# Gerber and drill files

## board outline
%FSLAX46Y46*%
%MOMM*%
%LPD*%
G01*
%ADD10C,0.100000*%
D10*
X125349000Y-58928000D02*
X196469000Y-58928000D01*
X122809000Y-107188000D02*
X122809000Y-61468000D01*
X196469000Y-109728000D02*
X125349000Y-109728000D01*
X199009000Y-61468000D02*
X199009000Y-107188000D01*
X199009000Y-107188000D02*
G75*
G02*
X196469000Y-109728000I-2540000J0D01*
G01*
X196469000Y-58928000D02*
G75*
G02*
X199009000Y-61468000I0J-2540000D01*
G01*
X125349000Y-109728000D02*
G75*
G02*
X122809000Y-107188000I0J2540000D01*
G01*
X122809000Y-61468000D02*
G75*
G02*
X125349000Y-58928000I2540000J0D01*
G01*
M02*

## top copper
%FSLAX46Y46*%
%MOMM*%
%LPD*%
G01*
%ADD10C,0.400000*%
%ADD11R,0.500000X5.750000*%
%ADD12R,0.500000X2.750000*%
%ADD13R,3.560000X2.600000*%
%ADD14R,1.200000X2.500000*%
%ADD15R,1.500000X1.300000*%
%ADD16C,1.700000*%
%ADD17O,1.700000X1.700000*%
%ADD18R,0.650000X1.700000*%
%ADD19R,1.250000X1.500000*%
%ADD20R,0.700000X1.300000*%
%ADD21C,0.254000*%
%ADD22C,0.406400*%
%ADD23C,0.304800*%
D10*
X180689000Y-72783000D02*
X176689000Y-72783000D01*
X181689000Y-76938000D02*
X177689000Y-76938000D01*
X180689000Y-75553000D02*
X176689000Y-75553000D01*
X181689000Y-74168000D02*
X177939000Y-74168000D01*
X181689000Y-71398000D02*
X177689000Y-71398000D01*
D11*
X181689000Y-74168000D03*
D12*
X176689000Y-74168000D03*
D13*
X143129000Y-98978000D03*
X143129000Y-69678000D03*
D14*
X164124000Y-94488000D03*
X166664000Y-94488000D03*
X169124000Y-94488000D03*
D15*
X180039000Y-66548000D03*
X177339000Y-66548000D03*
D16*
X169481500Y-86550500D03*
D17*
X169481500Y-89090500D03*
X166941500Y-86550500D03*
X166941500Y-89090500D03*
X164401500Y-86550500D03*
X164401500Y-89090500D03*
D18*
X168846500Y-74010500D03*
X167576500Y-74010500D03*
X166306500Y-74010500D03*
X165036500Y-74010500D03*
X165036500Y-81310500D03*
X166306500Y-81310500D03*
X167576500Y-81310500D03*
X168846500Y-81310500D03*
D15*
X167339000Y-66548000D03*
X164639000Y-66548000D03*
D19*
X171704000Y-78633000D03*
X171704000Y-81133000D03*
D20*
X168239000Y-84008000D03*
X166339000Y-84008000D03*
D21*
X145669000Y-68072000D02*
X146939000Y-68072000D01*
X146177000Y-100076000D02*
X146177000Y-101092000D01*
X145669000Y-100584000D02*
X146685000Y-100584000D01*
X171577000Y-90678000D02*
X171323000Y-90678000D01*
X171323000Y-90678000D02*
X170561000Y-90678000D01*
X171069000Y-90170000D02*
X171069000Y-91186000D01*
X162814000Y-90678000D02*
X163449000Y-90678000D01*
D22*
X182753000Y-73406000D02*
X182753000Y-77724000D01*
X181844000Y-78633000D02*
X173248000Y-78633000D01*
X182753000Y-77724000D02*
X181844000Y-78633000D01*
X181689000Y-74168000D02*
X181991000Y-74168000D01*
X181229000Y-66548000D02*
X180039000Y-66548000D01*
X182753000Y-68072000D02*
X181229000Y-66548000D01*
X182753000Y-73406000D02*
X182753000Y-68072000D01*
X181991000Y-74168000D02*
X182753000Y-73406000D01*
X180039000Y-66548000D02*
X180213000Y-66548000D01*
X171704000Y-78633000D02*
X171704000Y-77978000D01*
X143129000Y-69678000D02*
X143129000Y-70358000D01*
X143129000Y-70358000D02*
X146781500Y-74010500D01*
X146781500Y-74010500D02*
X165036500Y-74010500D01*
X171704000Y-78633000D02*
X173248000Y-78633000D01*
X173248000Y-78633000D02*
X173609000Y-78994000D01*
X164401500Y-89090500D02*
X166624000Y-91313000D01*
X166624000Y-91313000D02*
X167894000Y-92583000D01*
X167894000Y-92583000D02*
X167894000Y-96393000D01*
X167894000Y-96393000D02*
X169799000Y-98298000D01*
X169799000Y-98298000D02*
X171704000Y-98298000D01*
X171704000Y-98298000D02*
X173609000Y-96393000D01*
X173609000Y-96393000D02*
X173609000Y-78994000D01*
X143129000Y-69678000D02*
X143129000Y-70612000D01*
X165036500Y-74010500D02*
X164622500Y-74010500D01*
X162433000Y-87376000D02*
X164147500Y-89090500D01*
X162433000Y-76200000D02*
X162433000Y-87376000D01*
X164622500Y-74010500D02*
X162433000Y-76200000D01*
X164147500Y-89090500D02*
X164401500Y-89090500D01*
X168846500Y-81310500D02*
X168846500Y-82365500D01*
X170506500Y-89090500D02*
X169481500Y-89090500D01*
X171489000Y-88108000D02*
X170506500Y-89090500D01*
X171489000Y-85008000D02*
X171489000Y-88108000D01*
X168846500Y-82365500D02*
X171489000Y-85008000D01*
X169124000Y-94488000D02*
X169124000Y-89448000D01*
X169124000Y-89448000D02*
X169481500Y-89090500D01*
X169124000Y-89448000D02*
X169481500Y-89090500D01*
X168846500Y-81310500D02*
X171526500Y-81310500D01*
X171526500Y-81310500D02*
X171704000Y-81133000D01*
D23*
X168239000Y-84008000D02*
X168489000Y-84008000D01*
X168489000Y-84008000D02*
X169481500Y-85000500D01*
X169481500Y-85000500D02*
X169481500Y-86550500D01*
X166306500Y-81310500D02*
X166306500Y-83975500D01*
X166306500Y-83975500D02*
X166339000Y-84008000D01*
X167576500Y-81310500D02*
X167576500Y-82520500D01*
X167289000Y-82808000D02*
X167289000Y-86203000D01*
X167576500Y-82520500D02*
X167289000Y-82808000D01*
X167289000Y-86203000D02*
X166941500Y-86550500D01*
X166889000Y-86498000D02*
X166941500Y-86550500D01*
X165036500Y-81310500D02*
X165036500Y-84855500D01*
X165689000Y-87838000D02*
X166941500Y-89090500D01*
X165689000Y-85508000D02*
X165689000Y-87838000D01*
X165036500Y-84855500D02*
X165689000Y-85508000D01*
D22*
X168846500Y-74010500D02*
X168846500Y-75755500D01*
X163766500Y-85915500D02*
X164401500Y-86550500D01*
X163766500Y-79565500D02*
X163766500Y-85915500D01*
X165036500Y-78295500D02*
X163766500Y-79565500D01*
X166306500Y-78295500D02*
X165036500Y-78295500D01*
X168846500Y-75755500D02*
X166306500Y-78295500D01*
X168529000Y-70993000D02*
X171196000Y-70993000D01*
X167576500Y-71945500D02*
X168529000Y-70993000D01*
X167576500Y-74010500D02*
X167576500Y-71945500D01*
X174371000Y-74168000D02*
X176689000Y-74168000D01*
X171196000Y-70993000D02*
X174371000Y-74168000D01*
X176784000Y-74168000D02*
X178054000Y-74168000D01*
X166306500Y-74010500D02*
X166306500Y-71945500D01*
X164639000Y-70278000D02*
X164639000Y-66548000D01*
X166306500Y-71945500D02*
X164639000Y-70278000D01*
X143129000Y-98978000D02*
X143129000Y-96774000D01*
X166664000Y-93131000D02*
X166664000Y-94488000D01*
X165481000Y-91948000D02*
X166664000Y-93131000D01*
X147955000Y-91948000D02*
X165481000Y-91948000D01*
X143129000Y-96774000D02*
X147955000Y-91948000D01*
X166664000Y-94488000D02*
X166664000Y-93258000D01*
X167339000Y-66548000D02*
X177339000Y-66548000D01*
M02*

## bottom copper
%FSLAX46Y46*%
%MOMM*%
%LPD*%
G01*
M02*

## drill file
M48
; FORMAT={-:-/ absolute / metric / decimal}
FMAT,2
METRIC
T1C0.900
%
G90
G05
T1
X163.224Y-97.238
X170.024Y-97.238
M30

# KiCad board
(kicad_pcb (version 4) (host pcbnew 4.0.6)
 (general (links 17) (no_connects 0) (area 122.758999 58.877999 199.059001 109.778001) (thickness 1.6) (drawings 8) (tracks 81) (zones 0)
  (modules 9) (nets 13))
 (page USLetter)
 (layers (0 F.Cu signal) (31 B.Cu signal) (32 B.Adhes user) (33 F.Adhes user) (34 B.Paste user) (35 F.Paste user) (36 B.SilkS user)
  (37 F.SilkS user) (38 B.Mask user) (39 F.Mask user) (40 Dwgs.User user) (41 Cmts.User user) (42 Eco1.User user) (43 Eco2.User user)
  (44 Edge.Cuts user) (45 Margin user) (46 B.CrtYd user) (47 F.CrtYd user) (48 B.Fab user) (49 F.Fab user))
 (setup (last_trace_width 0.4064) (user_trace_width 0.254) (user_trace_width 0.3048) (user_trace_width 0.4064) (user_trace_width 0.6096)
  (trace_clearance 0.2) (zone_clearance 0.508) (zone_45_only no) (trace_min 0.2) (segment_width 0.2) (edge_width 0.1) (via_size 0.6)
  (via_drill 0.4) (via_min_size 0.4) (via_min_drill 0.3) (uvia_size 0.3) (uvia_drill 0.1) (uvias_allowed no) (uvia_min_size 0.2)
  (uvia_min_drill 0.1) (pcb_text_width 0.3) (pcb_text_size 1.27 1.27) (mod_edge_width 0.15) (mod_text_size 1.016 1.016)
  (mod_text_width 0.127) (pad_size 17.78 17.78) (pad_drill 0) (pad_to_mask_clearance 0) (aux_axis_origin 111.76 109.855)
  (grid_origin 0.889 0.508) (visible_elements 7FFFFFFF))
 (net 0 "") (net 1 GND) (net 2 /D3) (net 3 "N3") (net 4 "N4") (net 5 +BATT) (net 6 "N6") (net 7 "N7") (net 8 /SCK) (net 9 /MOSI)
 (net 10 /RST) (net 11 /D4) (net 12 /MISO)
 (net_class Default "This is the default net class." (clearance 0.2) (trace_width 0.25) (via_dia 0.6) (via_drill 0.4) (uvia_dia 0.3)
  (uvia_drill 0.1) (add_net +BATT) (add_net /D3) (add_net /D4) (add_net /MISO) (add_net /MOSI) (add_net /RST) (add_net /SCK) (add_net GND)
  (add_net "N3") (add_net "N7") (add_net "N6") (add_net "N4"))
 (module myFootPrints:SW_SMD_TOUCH (layer F.Cu) (at 178.689 74.168 270)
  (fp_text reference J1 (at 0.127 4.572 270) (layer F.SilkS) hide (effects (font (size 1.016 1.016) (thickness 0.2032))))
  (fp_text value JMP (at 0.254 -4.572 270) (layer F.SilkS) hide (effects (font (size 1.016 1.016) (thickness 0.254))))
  (fp_line (start -1.385 -2) (end -1.385 2) (layer F.Cu) (width 0.4))
  (fp_line (start 2.77 -3) (end 2.77 1) (layer F.Cu) (width 0.4))
  (fp_line (start 1.385 -2) (end 1.385 2) (layer F.Cu) (width 0.4)) (fp_line (start 0 -3) (end 0 0.75) (layer F.Cu) (width 0.4))
  (fp_line (start -2.77 -3) (end -2.77 1) (layer F.Cu) (width 0.4))
  (pad 1 smd rect (at 0 -3 270) (size 5.75 0.5) (layers F.Cu F.Paste F.Mask) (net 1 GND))
  (pad 2 smd rect (at 0 2 270) (size 2.75 0.5) (layers F.Cu F.Paste F.Mask) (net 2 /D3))
  (pad 3 smd circle (at 0 -1 270) (size 3.5 3.5) (layers F.Paste F.Mask)))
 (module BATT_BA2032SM (layer F.Cu) (at 143.129 84.328 90)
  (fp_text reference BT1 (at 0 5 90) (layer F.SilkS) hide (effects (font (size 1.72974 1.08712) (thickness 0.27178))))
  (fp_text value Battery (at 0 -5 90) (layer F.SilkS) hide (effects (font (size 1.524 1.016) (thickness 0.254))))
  (pad 1 smd rect (at -14.65 0 90) (size 2.6 3.56) (layers F.Cu F.Paste F.Mask) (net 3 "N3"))
  (pad 2 smd rect (at 14.65 0 90) (size 2.6 3.56) (layers F.Cu F.Paste F.Mask) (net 1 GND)))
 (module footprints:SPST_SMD (layer F.Cu) (at 166.624 94.488)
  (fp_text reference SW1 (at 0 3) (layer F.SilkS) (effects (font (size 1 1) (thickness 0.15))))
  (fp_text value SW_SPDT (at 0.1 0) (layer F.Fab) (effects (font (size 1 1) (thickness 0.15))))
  (pad "" np_thru_hole circle (at 3.4 2.75) (size 0.9 0.9) (drill 0.9) (layers *.Cu *.Mask))
  (pad 1 smd rect (at -2.5 0) (size 1.2 2.5) (layers F.Cu F.Paste F.Mask) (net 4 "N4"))
  (pad 2 smd rect (at 0.04 0) (size 1.2 2.5) (layers F.Cu F.Paste F.Mask) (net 3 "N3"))
  (pad 3 smd rect (at 2.5 0) (size 1.2 2.5) (layers F.Cu F.Paste F.Mask) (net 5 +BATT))
  (pad "" np_thru_hole circle (at -3.4 2.75) (size 0.9 0.9) (drill 0.9) (layers *.Cu *.Mask)))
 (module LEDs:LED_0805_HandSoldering (layer F.Cu) (at 178.689 66.548 180)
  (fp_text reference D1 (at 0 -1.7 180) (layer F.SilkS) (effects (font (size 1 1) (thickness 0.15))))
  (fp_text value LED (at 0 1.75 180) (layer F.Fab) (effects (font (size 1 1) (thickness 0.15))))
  (pad 1 smd rect (at -1.35 0 180) (size 1.5 1.3) (layers F.Cu F.Paste F.Mask) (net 1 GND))
  (pad 2 smd rect (at 1.35 0 180) (size 1.5 1.3) (layers F.Cu F.Paste F.Mask) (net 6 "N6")))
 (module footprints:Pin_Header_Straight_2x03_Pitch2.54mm (layer F.Cu) (at 169.4815 86.5505 270)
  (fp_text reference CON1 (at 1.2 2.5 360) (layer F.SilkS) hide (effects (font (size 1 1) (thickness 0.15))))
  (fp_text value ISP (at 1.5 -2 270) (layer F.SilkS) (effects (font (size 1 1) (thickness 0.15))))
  (pad 1 smd circle (at 0 0 270) (size 1.7 1.7) (layers F.Cu F.Paste F.Mask) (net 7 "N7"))
  (pad 2 smd oval (at 2.54 0 270) (size 1.7 1.7) (layers F.Cu F.Paste F.Mask) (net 5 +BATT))
  (pad 3 smd oval (at 0 2.54 270) (size 1.7 1.7) (layers F.Cu F.Paste F.Mask) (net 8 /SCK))
  (pad 4 smd oval (at 2.54 2.54 270) (size 1.7 1.7) (layers F.Cu F.Paste F.Mask) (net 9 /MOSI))
  (pad 5 smd oval (at 0 5.08 270) (size 1.7 1.7) (layers F.Cu F.Paste F.Mask) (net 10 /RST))
  (pad 6 smd oval (at 2.54 5.08 270) (size 1.7 1.7) (layers F.Cu F.Paste F.Mask) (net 1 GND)))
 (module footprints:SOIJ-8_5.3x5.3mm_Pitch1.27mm (layer F.Cu) (at 166.9415 77.6605 270)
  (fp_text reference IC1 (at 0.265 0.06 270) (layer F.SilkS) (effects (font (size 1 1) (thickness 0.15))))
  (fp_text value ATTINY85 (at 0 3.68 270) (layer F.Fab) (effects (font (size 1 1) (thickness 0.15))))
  (pad 1 smd rect (at -3.65 -1.905 270) (size 1.7 0.65) (layers F.Cu F.Paste F.Mask) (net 10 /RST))
  (pad 2 smd rect (at -3.65 -0.635 270) (size 1.7 0.65) (layers F.Cu F.Paste F.Mask) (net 2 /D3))
  (pad 3 smd rect (at -3.65 0.635 270) (size 1.7 0.65) (layers F.Cu F.Paste F.Mask) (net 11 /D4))
  (pad 4 smd rect (at -3.65 1.905 270) (size 1.7 0.65) (layers F.Cu F.Paste F.Mask) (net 1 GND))
  (pad 5 smd rect (at 3.65 1.905 270) (size 1.7 0.65) (layers F.Cu F.Paste F.Mask) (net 9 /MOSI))
  (pad 6 smd rect (at 3.65 0.635 270) (size 1.7 0.65) (layers F.Cu F.Paste F.Mask) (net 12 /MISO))
  (pad 7 smd rect (at 3.65 -0.635 270) (size 1.7 0.65) (layers F.Cu F.Paste F.Mask) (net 8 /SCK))
  (pad 8 smd rect (at 3.65 -1.905 270) (size 1.7 0.65) (layers F.Cu F.Paste F.Mask) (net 5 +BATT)))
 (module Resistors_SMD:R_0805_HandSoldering (layer F.Cu) (at 165.989 66.548 180)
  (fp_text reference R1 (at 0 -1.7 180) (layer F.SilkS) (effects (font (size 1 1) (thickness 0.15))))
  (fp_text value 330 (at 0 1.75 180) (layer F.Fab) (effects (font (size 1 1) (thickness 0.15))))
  (pad 1 smd rect (at -1.35 0 180) (size 1.5 1.3) (layers F.Cu F.Paste F.Mask) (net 6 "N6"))
  (pad 2 smd rect (at 1.35 0 180) (size 1.5 1.3) (layers F.Cu F.Paste F.Mask) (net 11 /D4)))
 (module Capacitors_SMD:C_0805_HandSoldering (layer F.Cu) (at 171.704 79.883 270)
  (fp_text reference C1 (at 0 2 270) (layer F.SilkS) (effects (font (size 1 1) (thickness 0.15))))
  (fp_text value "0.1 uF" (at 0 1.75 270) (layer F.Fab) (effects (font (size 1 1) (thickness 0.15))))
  (pad 1 smd rect (at -1.25 0 270) (size 1.5 1.25) (layers F.Cu F.Paste F.Mask) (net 1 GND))
  (pad 2 smd rect (at 1.25 0 270) (size 1.5 1.25) (layers F.Cu F.Paste F.Mask) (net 5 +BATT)))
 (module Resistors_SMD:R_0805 (layer F.Cu) (at 167.289 84.008 180)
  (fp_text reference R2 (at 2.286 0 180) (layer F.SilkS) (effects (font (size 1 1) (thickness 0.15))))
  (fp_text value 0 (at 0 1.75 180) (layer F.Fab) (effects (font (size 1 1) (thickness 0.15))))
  (pad 1 smd rect (at -0.95 0 180) (size 0.7 1.3) (layers F.Cu F.Paste F.Mask) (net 7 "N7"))
  (pad 2 smd rect (at 0.95 0 180) (size 0.7 1.3) (layers F.Cu F.Paste F.Mask) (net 12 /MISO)))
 (gr_line (start 125.349 58.928) (end 196.469 58.928) (angle 90) (layer Edge.Cuts) (width 0.1))
 (gr_line (start 122.809 107.188) (end 122.809 61.468) (angle 90) (layer Edge.Cuts) (width 0.1))
 (gr_line (start 196.469 109.728) (end 125.349 109.728) (angle 90) (layer Edge.Cuts) (width 0.1))
 (gr_line (start 199.009 61.468) (end 199.009 107.188) (angle 90) (layer Edge.Cuts) (width 0.1))
 (gr_arc (start 196.469 107.188) (end 199.009 107.188) (angle 90) (layer Edge.Cuts) (width 0.1))
 (gr_arc (start 196.469 61.468) (end 196.469 58.928) (angle 90) (layer Edge.Cuts) (width 0.1))
 (gr_arc (start 125.349 107.188) (end 125.349 109.728) (angle 90) (layer Edge.Cuts) (width 0.1))
 (gr_arc (start 125.349 61.468) (end 122.809 61.468) (angle 90) (layer Edge.Cuts) (width 0.1))
 (segment (start 145.669 68.072) (end 146.939 68.072) (width 0.254) (layer F.Cu) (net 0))
 (segment (start 146.177 100.076) (end 146.177 101.092) (width 0.254) (layer F.Cu) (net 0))
 (segment (start 145.669 100.584) (end 146.685 100.584) (width 0.254) (layer F.Cu) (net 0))
 (segment (start 171.577 90.678) (end 171.323 90.678) (width 0.254) (layer F.Cu) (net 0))
 (segment (start 171.323 90.678) (end 170.561 90.678) (width 0.254) (layer F.Cu) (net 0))
 (segment (start 171.069 90.17) (end 171.069 91.186) (width 0.254) (layer F.Cu) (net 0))
 (segment (start 162.814 90.678) (end 163.449 90.678) (width 0.254) (layer F.Cu) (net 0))
 (segment (start 182.753 73.406) (end 182.753 77.724) (width 0.4064) (layer F.Cu) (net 1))
 (segment (start 181.844 78.633) (end 173.248 78.633) (width 0.4064) (layer F.Cu) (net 1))
 (segment (start 182.753 77.724) (end 181.844 78.633) (width 0.4064) (layer F.Cu) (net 1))
 (segment (start 181.689 74.168) (end 181.991 74.168) (width 0.4064) (layer F.Cu) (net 1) (status 400000))
 (segment (start 181.229 66.548) (end 180.039 66.548) (width 0.4064) (layer F.Cu) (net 1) (status 800000))
 (segment (start 182.753 68.072) (end 181.229 66.548) (width 0.4064) (layer F.Cu) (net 1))
 (segment (start 182.753 73.406) (end 182.753 68.072) (width 0.4064) (layer F.Cu) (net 1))
 (segment (start 181.991 74.168) (end 182.753 73.406) (width 0.4064) (layer F.Cu) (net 1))
 (segment (start 180.039 66.548) (end 180.213 66.548) (width 0.4064) (layer F.Cu) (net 1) (status C00000))
 (segment (start 171.704 78.633) (end 171.704 77.978) (width 0.4064) (layer F.Cu) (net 1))
 (segment (start 143.129 69.678) (end 143.129 70.358) (width 0.4064) (layer F.Cu) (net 1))
 (segment (start 143.129 70.358) (end 146.7815 74.0105) (width 0.4064) (layer F.Cu) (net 1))
 (segment (start 146.7815 74.0105) (end 165.0365 74.0105) (width 0.4064) (layer F.Cu) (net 1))
 (segment (start 171.704 78.633) (end 173.248 78.633) (width 0.4064) (layer F.Cu) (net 1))
 (segment (start 173.248 78.633) (end 173.609 78.994) (width 0.4064) (layer F.Cu) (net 1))
 (segment (start 164.4015 89.0905) (end 166.624 91.313) (width 0.4064) (layer F.Cu) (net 1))
 (segment (start 166.624 91.313) (end 167.894 92.583) (width 0.4064) (layer F.Cu) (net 1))
 (segment (start 167.894 92.583) (end 167.894 96.393) (width 0.4064) (layer F.Cu) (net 1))
 (segment (start 167.894 96.393) (end 169.799 98.298) (width 0.4064) (layer F.Cu) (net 1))
 (segment (start 169.799 98.298) (end 171.704 98.298) (width 0.4064) (layer F.Cu) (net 1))
 (segment (start 171.704 98.298) (end 173.609 96.393) (width 0.4064) (layer F.Cu) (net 1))
 (segment (start 173.609 96.393) (end 173.609 78.994) (width 0.4064) (layer F.Cu) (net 1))
 (segment (start 143.129 69.678) (end 143.129 70.612) (width 0.4064) (layer F.Cu) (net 1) (status 30))
 (segment (start 165.0365 74.0105) (end 164.6225 74.0105) (width 0.4064) (layer F.Cu) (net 1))
 (segment (start 162.433 87.376) (end 164.1475 89.0905) (width 0.4064) (layer F.Cu) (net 1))
 (segment (start 162.433 76.2) (end 162.433 87.376) (width 0.4064) (layer F.Cu) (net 1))
 (segment (start 164.6225 74.0105) (end 162.433 76.2) (width 0.4064) (layer F.Cu) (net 1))
 (segment (start 164.1475 89.0905) (end 164.4015 89.0905) (width 0.4064) (layer F.Cu) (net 1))
 (segment (start 168.8465 81.3105) (end 168.8465 82.3655) (width 0.4064) (layer F.Cu) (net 5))
 (segment (start 170.5065 89.0905) (end 169.4815 89.0905) (width 0.4064) (layer F.Cu) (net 5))
 (segment (start 171.489 88.108) (end 170.5065 89.0905) (width 0.4064) (layer F.Cu) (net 5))
 (segment (start 171.489 85.008) (end 171.489 88.108) (width 0.4064) (layer F.Cu) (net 5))
 (segment (start 168.8465 82.3655) (end 171.489 85.008) (width 0.4064) (layer F.Cu) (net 5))
 (segment (start 169.124 94.488) (end 169.124 89.448) (width 0.4064) (layer F.Cu) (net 5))
 (segment (start 169.124 89.448) (end 169.4815 89.0905) (width 0.4064) (layer F.Cu) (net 5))
 (segment (start 169.124 89.448) (end 169.4815 89.0905) (width 0.4064) (layer F.Cu) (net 5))
 (segment (start 168.8465 81.3105) (end 171.5265 81.3105) (width 0.4064) (layer F.Cu) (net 5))
 (segment (start 171.5265 81.3105) (end 171.704 81.133) (width 0.4064) (layer F.Cu) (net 5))
 (segment (start 168.239 84.008) (end 168.489 84.008) (width 0.3048) (layer F.Cu) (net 7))
 (segment (start 168.489 84.008) (end 169.4815 85.0005) (width 0.3048) (layer F.Cu) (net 7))
 (segment (start 169.4815 85.0005) (end 169.4815 86.5505) (width 0.3048) (layer F.Cu) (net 7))
 (segment (start 166.3065 81.3105) (end 166.3065 83.9755) (width 0.3048) (layer F.Cu) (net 12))
 (segment (start 166.3065 83.9755) (end 166.339 84.008) (width 0.3048) (layer F.Cu) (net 12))
 (segment (start 167.5765 81.3105) (end 167.5765 82.5205) (width 0.3048) (layer F.Cu) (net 8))
 (segment (start 167.289 82.808) (end 167.289 86.203) (width 0.3048) (layer F.Cu) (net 8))
 (segment (start 167.5765 82.5205) (end 167.289 82.808) (width 0.3048) (layer F.Cu) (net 8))
 (segment (start 167.289 86.203) (end 166.9415 86.5505) (width 0.3048) (layer F.Cu) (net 8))
 (segment (start 166.889 86.498) (end 166.9415 86.5505) (width 0.3048) (layer F.Cu) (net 8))
 (segment (start 165.0365 81.3105) (end 165.0365 84.8555) (width 0.3048) (layer F.Cu) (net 9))
 (segment (start 165.689 87.838) (end 166.9415 89.0905) (width 0.3048) (layer F.Cu) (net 9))
 (segment (start 165.689 85.508) (end 165.689 87.838) (width 0.3048) (layer F.Cu) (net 9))
 (segment (start 165.0365 84.8555) (end 165.689 85.508) (width 0.3048) (layer F.Cu) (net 9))
 (segment (start 168.8465 74.0105) (end 168.8465 75.7555) (width 0.4064) (layer F.Cu) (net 10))
 (segment (start 163.7665 85.9155) (end 164.4015 86.5505) (width 0.4064) (layer F.Cu) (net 10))
 (segment (start 163.7665 79.5655) (end 163.7665 85.9155) (width 0.4064) (layer F.Cu) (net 10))
 (segment (start 165.0365 78.2955) (end 163.7665 79.5655) (width 0.4064) (layer F.Cu) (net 10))
 (segment (start 166.3065 78.2955) (end 165.0365 78.2955) (width 0.4064) (layer F.Cu) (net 10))
 (segment (start 168.8465 75.7555) (end 166.3065 78.2955) (width 0.4064) (layer F.Cu) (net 10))
 (segment (start 168.529 70.993) (end 171.196 70.993) (width 0.4064) (layer F.Cu) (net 2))
 (segment (start 167.5765 71.9455) (end 168.529 70.993) (width 0.4064) (layer F.Cu) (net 2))
 (segment (start 167.5765 74.0105) (end 167.5765 71.9455) (width 0.4064) (layer F.Cu) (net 2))
 (segment (start 174.371 74.168) (end 176.689 74.168) (width 0.4064) (layer F.Cu) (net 2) (status 800000))
 (segment (start 171.196 70.993) (end 174.371 74.168) (width 0.4064) (layer F.Cu) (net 2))
 (segment (start 176.784 74.168) (end 178.054 74.168) (width 0.4064) (layer F.Cu) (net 2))
 (segment (start 166.3065 74.0105) (end 166.3065 71.9455) (width 0.4064) (layer F.Cu) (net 11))
 (segment (start 164.639 70.278) (end 164.639 66.548) (width 0.4064) (layer F.Cu) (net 11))
 (segment (start 166.3065 71.9455) (end 164.639 70.278) (width 0.4064) (layer F.Cu) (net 11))
 (segment (start 143.129 98.978) (end 143.129 96.774) (width 0.4064) (layer F.Cu) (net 3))
 (segment (start 166.664 93.131) (end 166.664 94.488) (width 0.4064) (layer F.Cu) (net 3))
 (segment (start 165.481 91.948) (end 166.664 93.131) (width 0.4064) (layer F.Cu) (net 3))
 (segment (start 147.955 91.948) (end 165.481 91.948) (width 0.4064) (layer F.Cu) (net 3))
 (segment (start 143.129 96.774) (end 147.955 91.948) (width 0.4064) (layer F.Cu) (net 3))
 (segment (start 166.664 94.488) (end 166.664 93.258) (width 0.4064) (layer F.Cu) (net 3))
 (segment (start 167.339 66.548) (end 177.339 66.548) (width 0.4064) (layer F.Cu) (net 6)))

